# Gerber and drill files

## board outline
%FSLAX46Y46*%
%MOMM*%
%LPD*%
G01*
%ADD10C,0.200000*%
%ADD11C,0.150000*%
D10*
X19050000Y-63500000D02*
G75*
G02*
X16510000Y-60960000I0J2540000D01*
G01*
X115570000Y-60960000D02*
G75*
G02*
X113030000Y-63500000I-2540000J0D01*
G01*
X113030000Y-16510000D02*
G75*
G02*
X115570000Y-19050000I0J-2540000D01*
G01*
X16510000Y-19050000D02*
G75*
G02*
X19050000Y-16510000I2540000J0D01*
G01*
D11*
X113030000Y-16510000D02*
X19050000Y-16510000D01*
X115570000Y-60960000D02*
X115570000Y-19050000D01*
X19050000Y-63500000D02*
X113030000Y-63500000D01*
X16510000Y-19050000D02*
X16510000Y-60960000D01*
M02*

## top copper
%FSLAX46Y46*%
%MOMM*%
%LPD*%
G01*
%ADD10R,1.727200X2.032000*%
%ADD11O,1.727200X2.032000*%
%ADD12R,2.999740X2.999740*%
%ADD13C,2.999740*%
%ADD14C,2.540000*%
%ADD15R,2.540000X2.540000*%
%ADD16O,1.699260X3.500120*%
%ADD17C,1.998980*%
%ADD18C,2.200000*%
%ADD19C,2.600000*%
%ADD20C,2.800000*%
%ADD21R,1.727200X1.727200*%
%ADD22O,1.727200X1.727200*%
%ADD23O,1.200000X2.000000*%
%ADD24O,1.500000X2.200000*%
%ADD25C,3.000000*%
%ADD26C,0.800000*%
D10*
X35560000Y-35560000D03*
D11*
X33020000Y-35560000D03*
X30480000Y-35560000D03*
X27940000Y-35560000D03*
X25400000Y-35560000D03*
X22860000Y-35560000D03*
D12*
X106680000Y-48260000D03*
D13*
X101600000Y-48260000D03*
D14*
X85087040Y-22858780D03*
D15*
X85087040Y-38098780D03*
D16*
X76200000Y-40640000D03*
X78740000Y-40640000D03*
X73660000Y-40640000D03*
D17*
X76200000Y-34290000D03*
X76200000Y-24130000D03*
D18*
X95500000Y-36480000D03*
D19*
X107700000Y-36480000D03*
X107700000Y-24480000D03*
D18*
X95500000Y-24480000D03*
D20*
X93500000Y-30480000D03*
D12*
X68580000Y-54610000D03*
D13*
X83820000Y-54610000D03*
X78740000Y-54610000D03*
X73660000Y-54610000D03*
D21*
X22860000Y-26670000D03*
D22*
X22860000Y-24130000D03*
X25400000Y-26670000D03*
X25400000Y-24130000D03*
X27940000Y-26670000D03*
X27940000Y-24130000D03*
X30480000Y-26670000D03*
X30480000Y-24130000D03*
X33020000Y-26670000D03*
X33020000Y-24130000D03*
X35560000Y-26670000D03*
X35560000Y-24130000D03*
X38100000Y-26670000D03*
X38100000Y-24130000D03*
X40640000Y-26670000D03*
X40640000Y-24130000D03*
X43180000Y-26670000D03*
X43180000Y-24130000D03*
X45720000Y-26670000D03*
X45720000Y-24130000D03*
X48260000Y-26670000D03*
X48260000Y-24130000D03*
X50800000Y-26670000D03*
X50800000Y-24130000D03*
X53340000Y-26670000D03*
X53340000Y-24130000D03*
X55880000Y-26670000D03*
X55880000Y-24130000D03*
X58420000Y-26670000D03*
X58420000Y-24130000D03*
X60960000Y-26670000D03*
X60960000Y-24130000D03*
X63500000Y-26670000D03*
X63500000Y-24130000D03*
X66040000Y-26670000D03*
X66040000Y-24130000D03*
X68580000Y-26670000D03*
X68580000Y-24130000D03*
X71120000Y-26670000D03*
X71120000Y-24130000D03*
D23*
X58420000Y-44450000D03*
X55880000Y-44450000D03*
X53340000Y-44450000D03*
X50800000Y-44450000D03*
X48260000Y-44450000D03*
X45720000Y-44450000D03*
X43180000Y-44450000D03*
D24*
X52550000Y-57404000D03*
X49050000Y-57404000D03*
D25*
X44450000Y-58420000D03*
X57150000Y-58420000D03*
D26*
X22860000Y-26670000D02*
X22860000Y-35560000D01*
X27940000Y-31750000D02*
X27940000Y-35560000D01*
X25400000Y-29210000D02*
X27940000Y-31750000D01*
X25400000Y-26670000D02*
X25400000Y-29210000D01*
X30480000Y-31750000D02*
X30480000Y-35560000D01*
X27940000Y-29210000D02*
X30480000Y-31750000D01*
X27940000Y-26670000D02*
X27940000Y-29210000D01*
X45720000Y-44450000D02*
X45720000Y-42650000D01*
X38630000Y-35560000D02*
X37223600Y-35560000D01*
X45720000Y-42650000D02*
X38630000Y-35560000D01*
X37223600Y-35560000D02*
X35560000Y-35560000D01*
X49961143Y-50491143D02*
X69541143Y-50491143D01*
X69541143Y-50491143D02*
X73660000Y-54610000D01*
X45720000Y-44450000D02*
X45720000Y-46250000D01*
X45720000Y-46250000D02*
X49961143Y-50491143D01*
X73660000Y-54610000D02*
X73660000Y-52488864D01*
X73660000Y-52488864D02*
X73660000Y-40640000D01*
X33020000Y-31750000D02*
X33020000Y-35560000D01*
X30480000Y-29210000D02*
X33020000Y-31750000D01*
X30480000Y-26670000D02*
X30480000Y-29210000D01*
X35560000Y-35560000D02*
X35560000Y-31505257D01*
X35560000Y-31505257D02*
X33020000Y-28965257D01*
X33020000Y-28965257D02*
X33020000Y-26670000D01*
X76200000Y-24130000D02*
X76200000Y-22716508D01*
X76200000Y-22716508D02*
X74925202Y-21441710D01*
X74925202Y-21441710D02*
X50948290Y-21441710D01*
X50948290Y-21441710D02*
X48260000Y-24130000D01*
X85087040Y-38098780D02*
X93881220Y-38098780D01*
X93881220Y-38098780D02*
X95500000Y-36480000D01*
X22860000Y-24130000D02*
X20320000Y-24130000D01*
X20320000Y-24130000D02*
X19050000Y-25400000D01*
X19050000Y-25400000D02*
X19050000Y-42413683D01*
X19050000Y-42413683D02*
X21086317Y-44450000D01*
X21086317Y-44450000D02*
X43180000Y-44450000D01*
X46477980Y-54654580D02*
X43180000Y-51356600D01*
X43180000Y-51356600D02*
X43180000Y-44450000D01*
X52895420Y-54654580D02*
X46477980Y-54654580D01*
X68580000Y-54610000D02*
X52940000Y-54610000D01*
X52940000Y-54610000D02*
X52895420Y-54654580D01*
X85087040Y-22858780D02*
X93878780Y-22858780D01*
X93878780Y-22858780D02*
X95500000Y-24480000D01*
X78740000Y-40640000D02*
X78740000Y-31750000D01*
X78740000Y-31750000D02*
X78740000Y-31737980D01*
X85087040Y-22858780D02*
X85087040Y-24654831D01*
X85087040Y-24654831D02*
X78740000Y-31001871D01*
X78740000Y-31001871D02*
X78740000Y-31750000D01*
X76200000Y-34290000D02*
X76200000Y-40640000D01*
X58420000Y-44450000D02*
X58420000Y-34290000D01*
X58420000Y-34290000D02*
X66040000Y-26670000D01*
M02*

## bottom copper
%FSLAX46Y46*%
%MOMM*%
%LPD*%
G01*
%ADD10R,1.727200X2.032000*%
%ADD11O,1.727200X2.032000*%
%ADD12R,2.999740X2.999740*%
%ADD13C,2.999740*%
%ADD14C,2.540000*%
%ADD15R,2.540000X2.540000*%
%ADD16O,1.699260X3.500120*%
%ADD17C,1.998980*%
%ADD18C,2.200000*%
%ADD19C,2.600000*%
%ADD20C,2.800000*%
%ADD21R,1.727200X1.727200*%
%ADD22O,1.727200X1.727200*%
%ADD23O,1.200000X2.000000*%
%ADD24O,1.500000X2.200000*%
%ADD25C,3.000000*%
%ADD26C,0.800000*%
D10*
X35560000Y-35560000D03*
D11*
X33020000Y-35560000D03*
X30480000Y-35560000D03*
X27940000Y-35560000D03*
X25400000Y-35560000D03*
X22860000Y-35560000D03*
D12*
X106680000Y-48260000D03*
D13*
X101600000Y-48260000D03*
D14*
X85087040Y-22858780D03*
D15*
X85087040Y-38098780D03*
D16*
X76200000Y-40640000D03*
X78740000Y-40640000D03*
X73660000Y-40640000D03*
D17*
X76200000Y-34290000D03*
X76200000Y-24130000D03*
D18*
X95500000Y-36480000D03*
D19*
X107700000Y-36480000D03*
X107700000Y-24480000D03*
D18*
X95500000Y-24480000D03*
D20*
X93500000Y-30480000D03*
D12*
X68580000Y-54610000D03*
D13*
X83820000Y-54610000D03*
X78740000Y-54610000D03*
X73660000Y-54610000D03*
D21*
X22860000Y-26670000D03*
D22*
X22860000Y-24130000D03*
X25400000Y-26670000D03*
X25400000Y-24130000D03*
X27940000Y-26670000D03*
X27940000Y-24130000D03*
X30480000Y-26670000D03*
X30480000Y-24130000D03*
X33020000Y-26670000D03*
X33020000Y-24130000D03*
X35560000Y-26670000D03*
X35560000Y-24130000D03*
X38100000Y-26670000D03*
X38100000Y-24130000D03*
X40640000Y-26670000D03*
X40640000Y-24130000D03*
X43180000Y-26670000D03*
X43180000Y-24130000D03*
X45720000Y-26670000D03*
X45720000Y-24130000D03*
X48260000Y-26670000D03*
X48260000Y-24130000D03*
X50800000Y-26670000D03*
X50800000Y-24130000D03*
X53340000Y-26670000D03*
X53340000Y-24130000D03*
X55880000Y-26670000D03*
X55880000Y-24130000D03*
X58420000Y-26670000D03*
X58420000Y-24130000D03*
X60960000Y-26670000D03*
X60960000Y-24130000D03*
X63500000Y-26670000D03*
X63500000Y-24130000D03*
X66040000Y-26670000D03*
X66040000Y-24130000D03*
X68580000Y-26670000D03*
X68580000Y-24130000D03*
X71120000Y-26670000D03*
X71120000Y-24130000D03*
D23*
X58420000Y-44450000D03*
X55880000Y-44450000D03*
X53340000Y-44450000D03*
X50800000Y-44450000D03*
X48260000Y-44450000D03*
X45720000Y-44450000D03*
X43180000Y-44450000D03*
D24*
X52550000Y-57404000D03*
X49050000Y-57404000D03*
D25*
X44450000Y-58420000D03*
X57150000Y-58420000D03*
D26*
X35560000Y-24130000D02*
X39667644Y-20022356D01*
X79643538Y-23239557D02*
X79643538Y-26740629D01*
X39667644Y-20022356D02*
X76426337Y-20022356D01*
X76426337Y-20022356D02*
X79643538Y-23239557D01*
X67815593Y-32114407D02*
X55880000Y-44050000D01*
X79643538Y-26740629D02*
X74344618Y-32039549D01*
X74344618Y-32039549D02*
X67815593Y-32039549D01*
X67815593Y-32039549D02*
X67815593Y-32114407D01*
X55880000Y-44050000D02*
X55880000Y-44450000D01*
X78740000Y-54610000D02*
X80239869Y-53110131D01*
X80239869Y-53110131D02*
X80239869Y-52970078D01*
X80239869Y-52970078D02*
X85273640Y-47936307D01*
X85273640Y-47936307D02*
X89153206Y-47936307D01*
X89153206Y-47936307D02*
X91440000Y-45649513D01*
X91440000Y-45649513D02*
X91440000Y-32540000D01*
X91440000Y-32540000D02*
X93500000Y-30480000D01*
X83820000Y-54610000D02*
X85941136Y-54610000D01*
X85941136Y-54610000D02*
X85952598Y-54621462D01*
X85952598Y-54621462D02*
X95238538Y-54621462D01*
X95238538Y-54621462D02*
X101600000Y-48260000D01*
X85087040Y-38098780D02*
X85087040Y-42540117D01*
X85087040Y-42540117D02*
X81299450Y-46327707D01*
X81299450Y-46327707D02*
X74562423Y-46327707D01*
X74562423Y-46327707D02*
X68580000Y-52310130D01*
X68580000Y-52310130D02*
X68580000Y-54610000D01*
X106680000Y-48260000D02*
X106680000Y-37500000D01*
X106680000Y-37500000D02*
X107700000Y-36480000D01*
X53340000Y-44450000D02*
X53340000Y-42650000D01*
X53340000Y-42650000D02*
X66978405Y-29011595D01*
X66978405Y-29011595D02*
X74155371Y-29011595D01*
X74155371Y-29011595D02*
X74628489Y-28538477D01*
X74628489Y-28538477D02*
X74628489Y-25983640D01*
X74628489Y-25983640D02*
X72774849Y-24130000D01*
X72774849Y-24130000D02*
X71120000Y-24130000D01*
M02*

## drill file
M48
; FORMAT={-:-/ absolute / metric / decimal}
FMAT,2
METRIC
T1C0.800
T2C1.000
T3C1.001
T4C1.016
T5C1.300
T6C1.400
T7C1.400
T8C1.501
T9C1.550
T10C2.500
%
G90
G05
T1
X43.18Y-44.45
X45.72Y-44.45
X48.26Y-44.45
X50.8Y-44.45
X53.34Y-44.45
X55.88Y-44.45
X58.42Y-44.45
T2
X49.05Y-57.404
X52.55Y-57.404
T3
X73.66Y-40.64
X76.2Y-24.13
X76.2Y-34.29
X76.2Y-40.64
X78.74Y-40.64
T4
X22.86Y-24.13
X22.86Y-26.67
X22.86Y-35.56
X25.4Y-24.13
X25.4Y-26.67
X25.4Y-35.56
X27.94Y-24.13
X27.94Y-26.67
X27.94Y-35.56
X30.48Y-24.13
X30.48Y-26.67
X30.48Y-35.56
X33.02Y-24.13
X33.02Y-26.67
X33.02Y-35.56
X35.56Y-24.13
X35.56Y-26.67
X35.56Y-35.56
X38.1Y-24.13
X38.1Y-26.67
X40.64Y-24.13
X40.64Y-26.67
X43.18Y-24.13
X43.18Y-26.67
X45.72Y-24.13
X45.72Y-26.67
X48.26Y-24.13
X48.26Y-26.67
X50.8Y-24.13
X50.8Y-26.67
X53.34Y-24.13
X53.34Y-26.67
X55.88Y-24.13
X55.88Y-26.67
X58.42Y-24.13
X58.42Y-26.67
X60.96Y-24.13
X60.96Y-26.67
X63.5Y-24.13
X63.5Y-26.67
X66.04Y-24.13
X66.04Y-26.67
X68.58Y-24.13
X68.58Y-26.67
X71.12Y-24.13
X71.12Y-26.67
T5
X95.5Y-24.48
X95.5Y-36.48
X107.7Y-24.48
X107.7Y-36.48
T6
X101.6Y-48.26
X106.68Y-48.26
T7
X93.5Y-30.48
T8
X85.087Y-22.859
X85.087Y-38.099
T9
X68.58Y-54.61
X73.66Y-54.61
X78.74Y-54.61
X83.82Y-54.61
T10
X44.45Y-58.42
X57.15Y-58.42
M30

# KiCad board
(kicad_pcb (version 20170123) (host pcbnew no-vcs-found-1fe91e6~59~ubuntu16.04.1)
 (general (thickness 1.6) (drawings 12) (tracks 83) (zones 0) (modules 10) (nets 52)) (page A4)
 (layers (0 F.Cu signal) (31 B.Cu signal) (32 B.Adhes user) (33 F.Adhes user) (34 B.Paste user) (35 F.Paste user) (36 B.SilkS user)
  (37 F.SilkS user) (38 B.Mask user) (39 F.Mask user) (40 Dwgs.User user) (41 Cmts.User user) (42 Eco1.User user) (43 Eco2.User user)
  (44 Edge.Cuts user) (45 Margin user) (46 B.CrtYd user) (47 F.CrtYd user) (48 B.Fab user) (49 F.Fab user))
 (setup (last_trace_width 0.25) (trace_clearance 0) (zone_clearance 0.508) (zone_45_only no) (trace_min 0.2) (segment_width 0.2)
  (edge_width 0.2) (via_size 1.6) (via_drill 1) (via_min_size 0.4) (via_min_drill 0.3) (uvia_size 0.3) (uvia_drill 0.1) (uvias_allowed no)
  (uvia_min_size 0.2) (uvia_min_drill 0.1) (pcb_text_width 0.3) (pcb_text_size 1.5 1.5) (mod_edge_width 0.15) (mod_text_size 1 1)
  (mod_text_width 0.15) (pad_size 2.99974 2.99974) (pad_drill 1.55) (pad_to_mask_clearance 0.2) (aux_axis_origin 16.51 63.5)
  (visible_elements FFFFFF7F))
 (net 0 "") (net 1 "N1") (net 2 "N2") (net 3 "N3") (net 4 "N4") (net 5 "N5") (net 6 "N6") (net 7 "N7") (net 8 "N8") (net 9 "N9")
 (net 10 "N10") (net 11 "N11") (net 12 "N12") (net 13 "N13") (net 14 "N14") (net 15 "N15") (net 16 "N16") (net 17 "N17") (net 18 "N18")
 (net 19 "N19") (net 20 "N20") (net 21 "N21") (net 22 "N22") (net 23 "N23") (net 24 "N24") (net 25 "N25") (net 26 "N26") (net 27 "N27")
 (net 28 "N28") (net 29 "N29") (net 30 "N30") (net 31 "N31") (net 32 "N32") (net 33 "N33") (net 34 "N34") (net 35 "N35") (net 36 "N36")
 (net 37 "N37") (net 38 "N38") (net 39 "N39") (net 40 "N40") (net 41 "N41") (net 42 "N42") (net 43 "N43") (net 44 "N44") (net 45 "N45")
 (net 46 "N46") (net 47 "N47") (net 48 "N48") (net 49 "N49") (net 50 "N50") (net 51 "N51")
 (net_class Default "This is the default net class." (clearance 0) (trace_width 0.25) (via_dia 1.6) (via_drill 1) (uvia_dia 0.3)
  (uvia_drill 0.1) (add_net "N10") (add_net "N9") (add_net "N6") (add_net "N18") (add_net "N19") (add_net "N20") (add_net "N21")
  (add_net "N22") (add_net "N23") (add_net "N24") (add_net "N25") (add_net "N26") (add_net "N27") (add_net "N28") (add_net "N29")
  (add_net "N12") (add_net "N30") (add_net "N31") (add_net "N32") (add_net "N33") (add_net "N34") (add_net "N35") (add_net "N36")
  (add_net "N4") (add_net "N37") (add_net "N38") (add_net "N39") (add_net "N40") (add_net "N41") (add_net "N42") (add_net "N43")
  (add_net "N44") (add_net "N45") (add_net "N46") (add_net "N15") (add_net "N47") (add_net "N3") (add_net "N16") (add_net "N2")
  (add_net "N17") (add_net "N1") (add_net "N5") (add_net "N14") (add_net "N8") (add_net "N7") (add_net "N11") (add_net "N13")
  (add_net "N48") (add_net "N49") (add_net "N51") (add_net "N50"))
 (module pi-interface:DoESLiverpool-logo (layer F.Cu) (at 24.13 53.34)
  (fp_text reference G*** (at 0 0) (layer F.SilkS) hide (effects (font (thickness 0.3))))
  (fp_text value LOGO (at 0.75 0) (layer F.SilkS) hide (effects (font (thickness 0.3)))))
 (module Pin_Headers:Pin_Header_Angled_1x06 (layer F.Cu) (at 35.56 35.56 270)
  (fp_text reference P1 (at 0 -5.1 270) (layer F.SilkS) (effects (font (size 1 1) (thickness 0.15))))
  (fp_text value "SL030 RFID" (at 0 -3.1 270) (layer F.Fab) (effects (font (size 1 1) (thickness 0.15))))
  (pad 1 thru_hole rect (at 0 0 270) (size 2.032 1.7272) (drill 1.016) (layers *.Cu *.Mask F.SilkS) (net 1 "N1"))
  (pad 2 thru_hole oval (at 0 2.54 270) (size 2.032 1.7272) (drill 1.016) (layers *.Cu *.Mask F.SilkS) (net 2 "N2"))
  (pad 3 thru_hole oval (at 0 5.08 270) (size 2.032 1.7272) (drill 1.016) (layers *.Cu *.Mask F.SilkS) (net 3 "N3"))
  (pad 4 thru_hole oval (at 0 7.62 270) (size 2.032 1.7272) (drill 1.016) (layers *.Cu *.Mask F.SilkS) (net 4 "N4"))
  (pad 5 thru_hole oval (at 0 10.16 270) (size 2.032 1.7272) (drill 1.016) (layers *.Cu *.Mask F.SilkS) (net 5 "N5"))
  (pad 6 thru_hole oval (at 0 12.7 270) (size 2.032 1.7272) (drill 1.016) (layers *.Cu *.Mask F.SilkS) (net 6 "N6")))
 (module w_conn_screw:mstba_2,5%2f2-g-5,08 (layer F.Cu) (at 104.14 48.26 180)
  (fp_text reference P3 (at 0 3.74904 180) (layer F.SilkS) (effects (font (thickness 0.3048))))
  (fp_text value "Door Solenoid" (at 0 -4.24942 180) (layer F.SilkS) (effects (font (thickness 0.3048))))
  (pad 1 thru_hole rect (at -2.54 0 180) (size 2.99974 2.99974) (drill 1.39954) (layers *.Cu *.Mask F.SilkS) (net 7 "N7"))
  (pad 2 thru_hole circle (at 2.54 0 180) (size 2.99974 2.99974) (drill 1.39954) (layers *.Cu *.Mask F.SilkS) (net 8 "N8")))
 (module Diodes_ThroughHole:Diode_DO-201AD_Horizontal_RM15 (layer F.Cu) (at 85.09 38.1 90)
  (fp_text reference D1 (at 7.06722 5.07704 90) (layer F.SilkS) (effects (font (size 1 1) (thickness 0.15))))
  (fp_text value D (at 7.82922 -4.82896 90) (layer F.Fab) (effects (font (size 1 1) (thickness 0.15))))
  (pad 2 thru_hole circle (at 15.24122 -0.00296 270) (size 2.54 2.54) (drill 1.50114) (layers *.Cu *.Mask F.SilkS) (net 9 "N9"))
  (pad 1 thru_hole rect (at 0.00122 -0.00296 270) (size 2.54 2.54) (drill 1.50114) (layers *.Cu *.Mask F.SilkS) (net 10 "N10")))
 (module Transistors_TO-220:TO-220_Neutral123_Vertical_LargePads (layer F.Cu) (at 76.2 40.64 180)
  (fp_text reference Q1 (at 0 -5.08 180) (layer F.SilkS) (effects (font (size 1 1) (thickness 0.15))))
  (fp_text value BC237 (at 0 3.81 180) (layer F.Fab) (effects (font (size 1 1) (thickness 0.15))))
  (pad 2 thru_hole oval (at 0 0 270) (size 3.50012 1.69926) (drill 1.00076) (layers *.Cu *.Mask F.SilkS) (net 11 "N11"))
  (pad 1 thru_hole oval (at -2.54 0 270) (size 3.50012 1.69926) (drill 1.00076) (layers *.Cu *.Mask F.SilkS) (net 9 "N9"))
  (pad 3 thru_hole oval (at 2.54 0 270) (size 3.50012 1.69926) (drill 1.00076) (layers *.Cu *.Mask F.SilkS) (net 1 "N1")))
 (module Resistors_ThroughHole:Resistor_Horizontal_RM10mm (layer F.Cu) (at 76.2 29.21 90)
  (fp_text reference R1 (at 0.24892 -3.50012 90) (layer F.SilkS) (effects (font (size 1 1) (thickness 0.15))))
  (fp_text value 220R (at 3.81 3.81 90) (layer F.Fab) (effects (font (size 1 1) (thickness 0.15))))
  (pad 1 thru_hole circle (at -5.08 0 90) (size 1.99898 1.99898) (drill 1.00076) (layers *.Cu *.SilkS *.Mask) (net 11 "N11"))
  (pad 2 thru_hole circle (at 5.08 0 90) (size 1.99898 1.99898) (drill 1.00076) (layers *.Cu *.SilkS *.Mask) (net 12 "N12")))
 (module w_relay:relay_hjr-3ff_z (layer F.Cu) (at 101.6 30.48 90)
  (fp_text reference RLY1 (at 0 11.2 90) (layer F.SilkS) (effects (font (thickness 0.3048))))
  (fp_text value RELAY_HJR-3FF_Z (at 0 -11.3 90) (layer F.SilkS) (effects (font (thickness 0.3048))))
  (pad 2 thru_hole circle (at -6 -6.1 90) (size 2.2 2.2) (drill 1.3) (layers *.Cu *.Mask) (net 10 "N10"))
  (pad 3 thru_hole circle (at -6 6.1 90) (size 2.6 2.6) (drill 1.3) (layers *.Cu *.Mask) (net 7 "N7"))
  (pad 4 thru_hole circle (at 6 6.1 90) (size 2.6 2.6) (drill 1.3) (layers *.Cu *.Mask) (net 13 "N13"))
  (pad 5 thru_hole circle (at 6 -6.1 90) (size 2.2 2.2) (drill 1.3) (layers *.Cu *.Mask) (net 9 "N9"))
  (pad 1 thru_hole circle (at 0 -8.1 90) (size 2.8 2.8) (drill 1.4) (layers *.Cu *.Mask) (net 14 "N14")))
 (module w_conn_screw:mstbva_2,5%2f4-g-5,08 (layer F.Cu) (at 76.2 54.61)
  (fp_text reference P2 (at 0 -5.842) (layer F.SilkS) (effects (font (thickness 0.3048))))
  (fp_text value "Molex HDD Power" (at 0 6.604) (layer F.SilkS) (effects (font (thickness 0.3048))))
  (pad 1 thru_hole rect (at -7.62 0) (size 2.99974 2.99974) (drill 1.55) (layers *.Cu *.Mask F.SilkS) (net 10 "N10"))
  (pad 4 thru_hole circle (at 7.62 0) (size 2.99974 2.99974) (drill 1.55) (layers *.Cu *.Mask F.SilkS) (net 8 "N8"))
  (pad 3 thru_hole circle (at 2.54 0) (size 2.99974 2.99974) (drill 1.55) (layers *.Cu *.Mask F.SilkS) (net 14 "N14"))
  (pad 2 thru_hole circle (at -2.54 0) (size 2.99974 2.99974) (drill 1.55) (layers *.Cu *.Mask F.SilkS) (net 1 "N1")))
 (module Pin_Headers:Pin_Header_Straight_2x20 (layer F.Cu) (at 22.86 26.67 90)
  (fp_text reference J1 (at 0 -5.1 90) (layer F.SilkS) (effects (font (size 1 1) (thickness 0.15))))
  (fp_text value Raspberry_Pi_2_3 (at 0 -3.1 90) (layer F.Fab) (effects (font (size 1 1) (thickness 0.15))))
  (pad 1 thru_hole rect (at 0 0 90) (size 1.7272 1.7272) (drill 1.016) (layers *.Cu *.Mask F.SilkS) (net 6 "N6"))
  (pad 2 thru_hole oval (at 2.54 0 90) (size 1.7272 1.7272) (drill 1.016) (layers *.Cu *.Mask F.SilkS) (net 10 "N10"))
  (pad 3 thru_hole oval (at 0 2.54 90) (size 1.7272 1.7272) (drill 1.016) (layers *.Cu *.Mask F.SilkS) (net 4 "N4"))
  (pad 4 thru_hole oval (at 2.54 2.54 90) (size 1.7272 1.7272) (drill 1.016) (layers *.Cu *.Mask F.SilkS) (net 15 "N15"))
  (pad 5 thru_hole oval (at 0 5.08 90) (size 1.7272 1.7272) (drill 1.016) (layers *.Cu *.Mask F.SilkS) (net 3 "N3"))
  (pad 6 thru_hole oval (at 2.54 5.08 90) (size 1.7272 1.7272) (drill 1.016) (layers *.Cu *.Mask F.SilkS) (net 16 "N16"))
  (pad 7 thru_hole oval (at 0 7.62 90) (size 1.7272 1.7272) (drill 1.016) (layers *.Cu *.Mask F.SilkS) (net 2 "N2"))
  (pad 8 thru_hole oval (at 2.54 7.62 90) (size 1.7272 1.7272) (drill 1.016) (layers *.Cu *.Mask F.SilkS) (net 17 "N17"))
  (pad 9 thru_hole oval (at 0 10.16 90) (size 1.7272 1.7272) (drill 1.016) (layers *.Cu *.Mask F.SilkS) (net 1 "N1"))
  (pad 10 thru_hole oval (at 2.54 10.16 90) (size 1.7272 1.7272) (drill 1.016) (layers *.Cu *.Mask F.SilkS) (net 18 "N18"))
  (pad 11 thru_hole oval (at 0 12.7 90) (size 1.7272 1.7272) (drill 1.016) (layers *.Cu *.Mask F.SilkS) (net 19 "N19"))
  (pad 12 thru_hole oval (at 2.54 12.7 90) (size 1.7272 1.7272) (drill 1.016) (layers *.Cu *.Mask F.SilkS) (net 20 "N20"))
  (pad 13 thru_hole oval (at 0 15.24 90) (size 1.7272 1.7272) (drill 1.016) (layers *.Cu *.Mask F.SilkS) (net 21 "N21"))
  (pad 14 thru_hole oval (at 2.54 15.24 90) (size 1.7272 1.7272) (drill 1.016) (layers *.Cu *.Mask F.SilkS) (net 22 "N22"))
  (pad 15 thru_hole oval (at 0 17.78 90) (size 1.7272 1.7272) (drill 1.016) (layers *.Cu *.Mask F.SilkS) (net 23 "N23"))
  (pad 16 thru_hole oval (at 2.54 17.78 90) (size 1.7272 1.7272) (drill 1.016) (layers *.Cu *.Mask F.SilkS) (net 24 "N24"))
  (pad 17 thru_hole oval (at 0 20.32 90) (size 1.7272 1.7272) (drill 1.016) (layers *.Cu *.Mask F.SilkS) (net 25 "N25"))
  (pad 18 thru_hole oval (at 2.54 20.32 90) (size 1.7272 1.7272) (drill 1.016) (layers *.Cu *.Mask F.SilkS) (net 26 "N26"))
  (pad 19 thru_hole oval (at 0 22.86 90) (size 1.7272 1.7272) (drill 1.016) (layers *.Cu *.Mask F.SilkS) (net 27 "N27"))
  (pad 20 thru_hole oval (at 2.54 22.86 90) (size 1.7272 1.7272) (drill 1.016) (layers *.Cu *.Mask F.SilkS) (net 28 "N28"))
  (pad 21 thru_hole oval (at 0 25.4 90) (size 1.7272 1.7272) (drill 1.016) (layers *.Cu *.Mask F.SilkS) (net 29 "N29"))
  (pad 22 thru_hole oval (at 2.54 25.4 90) (size 1.7272 1.7272) (drill 1.016) (layers *.Cu *.Mask F.SilkS) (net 12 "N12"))
  (pad 23 thru_hole oval (at 0 27.94 90) (size 1.7272 1.7272) (drill 1.016) (layers *.Cu *.Mask F.SilkS) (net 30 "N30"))
  (pad 24 thru_hole oval (at 2.54 27.94 90) (size 1.7272 1.7272) (drill 1.016) (layers *.Cu *.Mask F.SilkS) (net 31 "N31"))
  (pad 25 thru_hole oval (at 0 30.48 90) (size 1.7272 1.7272) (drill 1.016) (layers *.Cu *.Mask F.SilkS) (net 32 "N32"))
  (pad 26 thru_hole oval (at 2.54 30.48 90) (size 1.7272 1.7272) (drill 1.016) (layers *.Cu *.Mask F.SilkS) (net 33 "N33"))
  (pad 27 thru_hole oval (at 0 33.02 90) (size 1.7272 1.7272) (drill 1.016) (layers *.Cu *.Mask F.SilkS) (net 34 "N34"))
  (pad 28 thru_hole oval (at 2.54 33.02 90) (size 1.7272 1.7272) (drill 1.016) (layers *.Cu *.Mask F.SilkS) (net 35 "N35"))
  (pad 29 thru_hole oval (at 0 35.56 90) (size 1.7272 1.7272) (drill 1.016) (layers *.Cu *.Mask F.SilkS) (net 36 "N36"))
  (pad 30 thru_hole oval (at 2.54 35.56 90) (size 1.7272 1.7272) (drill 1.016) (layers *.Cu *.Mask F.SilkS) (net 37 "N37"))
  (pad 31 thru_hole oval (at 0 38.1 90) (size 1.7272 1.7272) (drill 1.016) (layers *.Cu *.Mask F.SilkS) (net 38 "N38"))
  (pad 32 thru_hole oval (at 2.54 38.1 90) (size 1.7272 1.7272) (drill 1.016) (layers *.Cu *.Mask F.SilkS) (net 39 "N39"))
  (pad 33 thru_hole oval (at 0 40.64 90) (size 1.7272 1.7272) (drill 1.016) (layers *.Cu *.Mask F.SilkS) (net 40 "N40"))
  (pad 34 thru_hole oval (at 2.54 40.64 90) (size 1.7272 1.7272) (drill 1.016) (layers *.Cu *.Mask F.SilkS) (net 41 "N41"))
  (pad 35 thru_hole oval (at 0 43.18 90) (size 1.7272 1.7272) (drill 1.016) (layers *.Cu *.Mask F.SilkS) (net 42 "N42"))
  (pad 36 thru_hole oval (at 2.54 43.18 90) (size 1.7272 1.7272) (drill 1.016) (layers *.Cu *.Mask F.SilkS) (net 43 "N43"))
  (pad 37 thru_hole oval (at 0 45.72 90) (size 1.7272 1.7272) (drill 1.016) (layers *.Cu *.Mask F.SilkS) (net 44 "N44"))
  (pad 38 thru_hole oval (at 2.54 45.72 90) (size 1.7272 1.7272) (drill 1.016) (layers *.Cu *.Mask F.SilkS) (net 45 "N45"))
  (pad 39 thru_hole oval (at 0 48.26 90) (size 1.7272 1.7272) (drill 1.016) (layers *.Cu *.Mask F.SilkS) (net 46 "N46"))
  (pad 40 thru_hole oval (at 2.54 48.26 90) (size 1.7272 1.7272) (drill 1.016) (layers *.Cu *.Mask F.SilkS) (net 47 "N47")))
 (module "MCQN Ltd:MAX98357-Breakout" (layer F.Cu) (at 50.8 44.45 180)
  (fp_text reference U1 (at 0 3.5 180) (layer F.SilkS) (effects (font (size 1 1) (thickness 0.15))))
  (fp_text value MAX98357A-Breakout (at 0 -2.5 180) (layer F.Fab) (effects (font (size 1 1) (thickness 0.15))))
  (pad 1 thru_hole oval (at -7.62 0 180) (size 1.2 2) (drill 0.8) (layers *.Cu *.Mask) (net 42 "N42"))
  (pad 2 thru_hole oval (at -5.08 0 180) (size 1.2 2) (drill 0.8) (layers *.Cu *.Mask) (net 20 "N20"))
  (pad 3 thru_hole oval (at -2.54 0 180) (size 1.2 2) (drill 0.8) (layers *.Cu *.Mask) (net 47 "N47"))
  (pad 4 thru_hole oval (at 0 0 180) (size 1.2 2) (drill 0.8) (layers *.Cu *.Mask) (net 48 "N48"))
  (pad 5 thru_hole oval (at 2.54 0 180) (size 1.2 2) (drill 0.8) (layers *.Cu *.Mask) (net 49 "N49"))
  (pad 6 thru_hole oval (at 5.08 0 180) (size 1.2 2) (drill 0.8) (layers *.Cu *.Mask) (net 1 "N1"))
  (pad 7 thru_hole oval (at 7.62 0 180) (size 1.2 2) (drill 0.8) (layers *.Cu *.Mask) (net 10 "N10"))
  (pad 9 thru_hole oval (at -1.75 -12.954 180) (size 1.5 2.2) (drill 1) (layers *.Cu *.Mask) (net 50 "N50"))
  (pad 8 thru_hole oval (at 1.75 -12.954 180) (size 1.5 2.2) (drill 1) (layers *.Cu *.Mask) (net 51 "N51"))
  (pad "" np_thru_hole circle (at 6.35 -13.97 180) (size 3 3) (drill 2.5) (layers *.Cu *.Mask))
  (pad "" np_thru_hole circle (at -6.35 -13.97 180) (size 3 3) (drill 2.5) (layers *.Cu *.Mask)))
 (gr_arc (start 19.05 60.96) (end 19.05 63.5) (angle 90) (layer Edge.Cuts) (width 0.2))
 (gr_arc (start 113.03 60.96) (end 113.03 63.5) (angle -90) (layer Edge.Cuts) (width 0.2))
 (gr_arc (start 113.03 19.05) (end 113.03 16.51) (angle 90) (layer Edge.Cuts) (width 0.2))
 (gr_arc (start 19.05 19.05) (end 16.51 19.05) (angle 90) (layer Edge.Cuts) (width 0.2))
 (gr_line (start 113.03 16.51) (end 19.05 16.51) (layer Edge.Cuts) (width 0.15))
 (gr_line (start 115.57 60.96) (end 115.57 19.05) (layer Edge.Cuts) (width 0.15))
 (gr_line (start 19.05 63.5) (end 113.03 63.5) (layer Edge.Cuts) (width 0.15))
 (gr_line (start 16.51 19.05) (end 16.51 60.96) (layer Edge.Cuts) (width 0.15))
 (segment (start 22.86 26.67) (end 22.86 35.56) (width 0.8) (layer F.Cu) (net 6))
 (segment (start 27.94 31.75) (end 27.94 35.56) (width 0.8) (layer F.Cu) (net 4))
 (segment (start 25.4 29.21) (end 27.94 31.75) (width 0.8) (layer F.Cu) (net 4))
 (segment (start 25.4 26.67) (end 25.4 29.21) (width 0.8) (layer F.Cu) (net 4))
 (segment (start 30.48 31.75) (end 30.48 35.56) (width 0.8) (layer F.Cu) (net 3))
 (segment (start 27.94 29.21) (end 30.48 31.75) (width 0.8) (layer F.Cu) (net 3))
 (segment (start 27.94 26.67) (end 27.94 29.21) (width 0.8) (layer F.Cu) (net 3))
 (segment (start 45.72 44.45) (end 45.72 42.65) (width 0.8) (layer F.Cu) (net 1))
 (segment (start 38.63 35.56) (end 37.2236 35.56) (width 0.8) (layer F.Cu) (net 1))
 (segment (start 45.72 42.65) (end 38.63 35.56) (width 0.8) (layer F.Cu) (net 1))
 (segment (start 37.2236 35.56) (end 35.56 35.56) (width 0.8) (layer F.Cu) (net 1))
 (segment (start 49.961143 50.491143) (end 69.541143 50.491143) (width 0.8) (layer F.Cu) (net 1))
 (segment (start 69.541143 50.491143) (end 73.66 54.61) (width 0.8) (layer F.Cu) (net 1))
 (segment (start 45.72 44.45) (end 45.72 46.25) (width 0.8) (layer F.Cu) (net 1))
 (segment (start 45.72 46.25) (end 49.961143 50.491143) (width 0.8) (layer F.Cu) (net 1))
 (segment (start 73.66 54.61) (end 73.66 52.488864) (width 0.8) (layer F.Cu) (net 1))
 (segment (start 73.66 52.488864) (end 73.66 40.64) (width 0.8) (layer F.Cu) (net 1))
 (segment (start 33.02 31.75) (end 33.02 35.56) (width 0.8) (layer F.Cu) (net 2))
 (segment (start 30.48 29.21) (end 33.02 31.75) (width 0.8) (layer F.Cu) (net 2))
 (segment (start 30.48 26.67) (end 30.48 29.21) (width 0.8) (layer F.Cu) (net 2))
 (segment (start 35.56 35.56) (end 35.56 31.505257) (width 0.8) (layer F.Cu) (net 1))
 (segment (start 35.56 31.505257) (end 33.02 28.965257) (width 0.8) (layer F.Cu) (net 1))
 (segment (start 33.02 28.965257) (end 33.02 26.67) (width 0.8) (layer F.Cu) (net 1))
 (segment (start 35.56 24.13) (end 39.667644 20.022356) (width 0.8) (layer B.Cu) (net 20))
 (segment (start 79.643538 23.239557) (end 79.643538 26.740629) (width 0.8) (layer B.Cu) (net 20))
 (segment (start 39.667644 20.022356) (end 76.426337 20.022356) (width 0.8) (layer B.Cu) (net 20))
 (segment (start 76.426337 20.022356) (end 79.643538 23.239557) (width 0.8) (layer B.Cu) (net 20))
 (segment (start 67.815593 32.114407) (end 55.88 44.05) (width 0.8) (layer B.Cu) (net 20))
 (segment (start 79.643538 26.740629) (end 74.344618 32.039549) (width 0.8) (layer B.Cu) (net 20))
 (segment (start 74.344618 32.039549) (end 67.815593 32.039549) (width 0.8) (layer B.Cu) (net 20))
 (segment (start 67.815593 32.039549) (end 67.815593 32.114407) (width 0.8) (layer B.Cu) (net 20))
 (segment (start 55.88 44.05) (end 55.88 44.45) (width 0.8) (layer B.Cu) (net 20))
 (segment (start 76.2 24.13) (end 76.2 22.716508) (width 0.8) (layer F.Cu) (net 12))
 (segment (start 76.2 22.716508) (end 74.925202 21.44171) (width 0.8) (layer F.Cu) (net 12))
 (segment (start 74.925202 21.44171) (end 50.94829 21.44171) (width 0.8) (layer F.Cu) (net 12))
 (segment (start 50.94829 21.44171) (end 48.26 24.13) (width 0.8) (layer F.Cu) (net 12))
 (segment (start 78.74 54.61) (end 80.239869 53.110131) (width 0.8) (layer B.Cu) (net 14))
 (segment (start 80.239869 53.110131) (end 80.239869 52.970078) (width 0.8) (layer B.Cu) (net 14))
 (segment (start 80.239869 52.970078) (end 85.27364 47.936307) (width 0.8) (layer B.Cu) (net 14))
 (segment (start 85.27364 47.936307) (end 89.153206 47.936307) (width 0.8) (layer B.Cu) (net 14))
 (segment (start 89.153206 47.936307) (end 91.44 45.649513) (width 0.8) (layer B.Cu) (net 14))
 (segment (start 91.44 45.649513) (end 91.44 32.54) (width 0.8) (layer B.Cu) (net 14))
 (segment (start 91.44 32.54) (end 93.5 30.48) (width 0.8) (layer B.Cu) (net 14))
 (segment (start 83.82 54.61) (end 85.941136 54.61) (width 0.8) (layer B.Cu) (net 8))
 (segment (start 85.941136 54.61) (end 85.952598 54.621462) (width 0.8) (layer B.Cu) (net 8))
 (segment (start 85.952598 54.621462) (end 95.238538 54.621462) (width 0.8) (layer B.Cu) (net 8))
 (segment (start 95.238538 54.621462) (end 101.6 48.26) (width 0.8) (layer B.Cu) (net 8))
 (segment (start 85.08704 38.09878) (end 93.88122 38.09878) (width 0.8) (layer F.Cu) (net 10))
 (segment (start 93.88122 38.09878) (end 95.5 36.48) (width 0.8) (layer F.Cu) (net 10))
 (segment (start 85.08704 38.09878) (end 85.08704 42.540117) (width 0.8) (layer B.Cu) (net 10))
 (segment (start 85.08704 42.540117) (end 81.29945 46.327707) (width 0.8) (layer B.Cu) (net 10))
 (segment (start 81.29945 46.327707) (end 74.562423 46.327707) (width 0.8) (layer B.Cu) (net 10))
 (segment (start 74.562423 46.327707) (end 68.58 52.31013) (width 0.8) (layer B.Cu) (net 10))
 (segment (start 68.58 52.31013) (end 68.58 54.61) (width 0.8) (layer B.Cu) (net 10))
 (segment (start 22.86 24.13) (end 20.32 24.13) (width 0.8) (layer F.Cu) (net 10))
 (segment (start 20.32 24.13) (end 19.05 25.4) (width 0.8) (layer F.Cu) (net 10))
 (segment (start 19.05 25.4) (end 19.05 42.413683) (width 0.8) (layer F.Cu) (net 10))
 (segment (start 19.05 42.413683) (end 21.086317 44.45) (width 0.8) (layer F.Cu) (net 10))
 (segment (start 21.086317 44.45) (end 43.18 44.45) (width 0.8) (layer F.Cu) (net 10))
 (segment (start 46.47798 54.65458) (end 43.18 51.3566) (width 0.8) (layer F.Cu) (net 10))
 (segment (start 43.18 51.3566) (end 43.18 44.45) (width 0.8) (layer F.Cu) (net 10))
 (segment (start 52.89542 54.65458) (end 46.47798 54.65458) (width 0.8) (layer F.Cu) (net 10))
 (segment (start 68.58 54.61) (end 52.94 54.61) (width 0.8) (layer F.Cu) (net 10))
 (segment (start 52.94 54.61) (end 52.89542 54.65458) (width 0.8) (layer F.Cu) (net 10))
 (segment (start 85.08704 22.85878) (end 93.87878 22.85878) (width 0.8) (layer F.Cu) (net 9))
 (segment (start 93.87878 22.85878) (end 95.5 24.48) (width 0.8) (layer F.Cu) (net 9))
 (segment (start 78.74 40.64) (end 78.74 31.75) (width 0.8) (layer F.Cu) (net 9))
 (segment (start 78.74 31.75) (end 78.74 31.73798) (width 0.8) (layer F.Cu) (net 9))
 (segment (start 85.08704 22.85878) (end 85.08704 24.654831) (width 0.8) (layer F.Cu) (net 9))
 (segment (start 85.08704 24.654831) (end 78.74 31.001871) (width 0.8) (layer F.Cu) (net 9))
 (segment (start 78.74 31.001871) (end 78.74 31.75) (width 0.8) (layer F.Cu) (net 9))
 (segment (start 76.2 34.29) (end 76.2 40.64) (width 0.8) (layer F.Cu) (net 11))
 (segment (start 106.68 48.26) (end 106.68 37.5) (width 0.8) (layer B.Cu) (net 7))
 (segment (start 106.68 37.5) (end 107.7 36.48) (width 0.8) (layer B.Cu) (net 7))
 (segment (start 58.42 44.45) (end 58.42 34.29) (width 0.8) (layer F.Cu) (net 42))
 (segment (start 58.42 34.29) (end 66.04 26.67) (width 0.8) (layer F.Cu) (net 42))
 (segment (start 53.34 44.45) (end 53.34 42.65) (width 0.8) (layer B.Cu) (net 47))
 (segment (start 53.34 42.65) (end 66.978405 29.011595) (width 0.8) (layer B.Cu) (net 47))
 (segment (start 66.978405 29.011595) (end 74.155371 29.011595) (width 0.8) (layer B.Cu) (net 47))
 (segment (start 74.155371 29.011595) (end 74.628489 28.538477) (width 0.8) (layer B.Cu) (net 47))
 (segment (start 74.628489 28.538477) (end 74.628489 25.98364) (width 0.8) (layer B.Cu) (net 47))
 (segment (start 74.628489 25.98364) (end 72.774849 24.13) (width 0.8) (layer B.Cu) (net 47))
 (segment (start 72.774849 24.13) (end 71.12 24.13) (width 0.8) (layer B.Cu) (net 47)))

